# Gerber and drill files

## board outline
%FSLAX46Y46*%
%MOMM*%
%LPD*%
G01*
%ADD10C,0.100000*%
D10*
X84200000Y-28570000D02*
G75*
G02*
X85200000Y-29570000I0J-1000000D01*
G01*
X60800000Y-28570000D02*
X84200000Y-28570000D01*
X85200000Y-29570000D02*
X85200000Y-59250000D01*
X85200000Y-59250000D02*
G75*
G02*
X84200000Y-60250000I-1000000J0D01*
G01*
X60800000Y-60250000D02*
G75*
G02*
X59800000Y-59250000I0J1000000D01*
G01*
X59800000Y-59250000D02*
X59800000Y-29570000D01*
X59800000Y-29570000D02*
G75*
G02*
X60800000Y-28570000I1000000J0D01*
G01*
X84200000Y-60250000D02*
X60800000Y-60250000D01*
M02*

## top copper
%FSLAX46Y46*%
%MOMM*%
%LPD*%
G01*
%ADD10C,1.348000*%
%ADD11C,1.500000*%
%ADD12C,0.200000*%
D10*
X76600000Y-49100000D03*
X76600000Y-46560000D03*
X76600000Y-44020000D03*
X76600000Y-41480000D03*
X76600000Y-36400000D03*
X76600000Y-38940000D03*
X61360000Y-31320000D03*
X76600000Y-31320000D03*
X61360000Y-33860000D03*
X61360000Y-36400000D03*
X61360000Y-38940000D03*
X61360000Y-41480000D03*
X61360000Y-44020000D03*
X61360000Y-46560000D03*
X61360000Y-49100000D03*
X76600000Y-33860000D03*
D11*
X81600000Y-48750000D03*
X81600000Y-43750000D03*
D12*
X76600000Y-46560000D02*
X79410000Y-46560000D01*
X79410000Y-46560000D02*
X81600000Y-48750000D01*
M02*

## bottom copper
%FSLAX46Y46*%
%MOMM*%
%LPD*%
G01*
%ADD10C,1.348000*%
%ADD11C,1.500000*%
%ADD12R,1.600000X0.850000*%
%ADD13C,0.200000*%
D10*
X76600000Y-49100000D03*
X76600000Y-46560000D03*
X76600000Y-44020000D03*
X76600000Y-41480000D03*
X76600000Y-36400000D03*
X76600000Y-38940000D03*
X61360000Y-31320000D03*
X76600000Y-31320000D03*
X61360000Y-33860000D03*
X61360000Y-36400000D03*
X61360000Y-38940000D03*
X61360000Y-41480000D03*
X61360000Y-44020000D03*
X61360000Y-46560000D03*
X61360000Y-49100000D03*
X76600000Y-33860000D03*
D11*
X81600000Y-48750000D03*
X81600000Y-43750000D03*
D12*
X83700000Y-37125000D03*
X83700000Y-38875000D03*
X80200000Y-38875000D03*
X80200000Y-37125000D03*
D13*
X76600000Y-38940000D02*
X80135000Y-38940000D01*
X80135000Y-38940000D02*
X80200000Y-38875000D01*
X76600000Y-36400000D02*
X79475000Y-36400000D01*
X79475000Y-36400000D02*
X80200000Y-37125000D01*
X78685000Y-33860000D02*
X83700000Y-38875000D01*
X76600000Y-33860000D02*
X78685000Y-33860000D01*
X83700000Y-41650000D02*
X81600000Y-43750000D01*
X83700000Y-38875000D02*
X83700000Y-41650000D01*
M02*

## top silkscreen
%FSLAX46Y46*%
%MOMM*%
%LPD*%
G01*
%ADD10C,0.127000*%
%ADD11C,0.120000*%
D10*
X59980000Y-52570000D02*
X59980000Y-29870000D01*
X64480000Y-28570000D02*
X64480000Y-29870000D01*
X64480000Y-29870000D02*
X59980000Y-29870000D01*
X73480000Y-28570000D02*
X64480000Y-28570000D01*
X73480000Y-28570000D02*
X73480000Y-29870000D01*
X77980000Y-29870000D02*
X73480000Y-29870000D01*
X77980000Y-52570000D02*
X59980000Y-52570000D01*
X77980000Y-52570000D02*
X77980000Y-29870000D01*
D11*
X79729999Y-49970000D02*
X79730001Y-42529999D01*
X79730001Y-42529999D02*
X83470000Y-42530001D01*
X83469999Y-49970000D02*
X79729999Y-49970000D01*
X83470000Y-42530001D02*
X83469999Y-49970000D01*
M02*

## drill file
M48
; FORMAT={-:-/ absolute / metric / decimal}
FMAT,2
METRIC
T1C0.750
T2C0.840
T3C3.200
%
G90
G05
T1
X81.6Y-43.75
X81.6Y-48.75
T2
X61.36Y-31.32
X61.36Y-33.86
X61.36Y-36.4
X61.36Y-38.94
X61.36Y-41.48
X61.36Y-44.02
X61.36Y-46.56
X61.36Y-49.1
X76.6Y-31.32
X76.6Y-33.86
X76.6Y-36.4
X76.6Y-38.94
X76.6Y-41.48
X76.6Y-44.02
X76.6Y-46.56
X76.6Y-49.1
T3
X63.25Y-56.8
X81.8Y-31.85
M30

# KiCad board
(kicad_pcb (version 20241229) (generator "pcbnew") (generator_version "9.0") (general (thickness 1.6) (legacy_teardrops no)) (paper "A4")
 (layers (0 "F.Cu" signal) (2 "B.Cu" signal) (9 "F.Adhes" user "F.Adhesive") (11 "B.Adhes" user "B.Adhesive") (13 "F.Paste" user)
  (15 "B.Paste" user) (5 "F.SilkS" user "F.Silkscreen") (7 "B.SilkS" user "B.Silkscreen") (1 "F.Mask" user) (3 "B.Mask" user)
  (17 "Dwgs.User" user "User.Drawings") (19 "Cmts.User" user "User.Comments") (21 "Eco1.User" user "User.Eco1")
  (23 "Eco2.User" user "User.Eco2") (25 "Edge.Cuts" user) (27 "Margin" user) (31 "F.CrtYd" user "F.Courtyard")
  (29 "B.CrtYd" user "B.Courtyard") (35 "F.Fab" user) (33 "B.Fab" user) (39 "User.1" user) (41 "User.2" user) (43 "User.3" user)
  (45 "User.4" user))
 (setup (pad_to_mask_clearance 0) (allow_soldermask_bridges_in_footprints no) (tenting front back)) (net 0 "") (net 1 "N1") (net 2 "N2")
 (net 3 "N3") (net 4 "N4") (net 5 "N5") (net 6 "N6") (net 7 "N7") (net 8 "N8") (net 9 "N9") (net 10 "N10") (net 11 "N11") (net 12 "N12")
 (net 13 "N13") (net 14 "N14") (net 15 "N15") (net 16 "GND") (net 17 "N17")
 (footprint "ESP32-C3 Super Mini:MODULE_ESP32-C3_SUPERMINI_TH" (layer "F.Cu") (at 68.98 41.22)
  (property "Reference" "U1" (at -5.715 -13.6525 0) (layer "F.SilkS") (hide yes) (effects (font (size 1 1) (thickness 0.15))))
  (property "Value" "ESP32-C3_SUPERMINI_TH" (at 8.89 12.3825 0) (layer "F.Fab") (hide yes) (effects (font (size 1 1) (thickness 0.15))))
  (fp_line (start -9 11.35) (end -9 -11.35) (stroke (width 0.127) (type solid)) (layer "F.SilkS"))
  (fp_line (start -4.5 -12.65) (end -4.5 -11.35) (stroke (width 0.127) (type solid)) (layer "F.SilkS"))
  (fp_line (start -4.5 -11.35) (end -9 -11.35) (stroke (width 0.127) (type solid)) (layer "F.SilkS"))
  (fp_line (start 4.5 -12.65) (end -4.5 -12.65) (stroke (width 0.127) (type solid)) (layer "F.SilkS"))
  (fp_line (start 4.5 -12.65) (end 4.5 -11.35) (stroke (width 0.127) (type solid)) (layer "F.SilkS"))
  (fp_line (start 9 -11.35) (end 4.5 -11.35) (stroke (width 0.127) (type solid)) (layer "F.SilkS"))
  (fp_line (start 9 11.35) (end -9 11.35) (stroke (width 0.127) (type solid)) (layer "F.SilkS"))
  (fp_line (start 9 11.35) (end 9 -11.35) (stroke (width 0.127) (type solid)) (layer "F.SilkS"))
  (pad "0" thru_hole circle (at 7.62 7.88) (size 1.348 1.348) (drill 0.84) (layers "*.Cu" "*.Mask") (remove_unused_layers no) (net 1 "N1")
   (solder_mask_margin 0.102))
  (pad "1" thru_hole circle (at 7.62 5.34) (size 1.348 1.348) (drill 0.84) (layers "*.Cu" "*.Mask") (remove_unused_layers no) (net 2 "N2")
   (solder_mask_margin 0.102))
  (pad "2" thru_hole circle (at 7.62 2.8) (size 1.348 1.348) (drill 0.84) (layers "*.Cu" "*.Mask") (remove_unused_layers no) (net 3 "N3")
   (solder_mask_margin 0.102))
  (pad "3" thru_hole circle (at 7.62 0.26) (size 1.348 1.348) (drill 0.84) (layers "*.Cu" "*.Mask") (remove_unused_layers no) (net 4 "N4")
   (solder_mask_margin 0.102))
  (pad "3.3" thru_hole circle (at 7.62 -4.82) (size 1.348 1.348) (drill 0.84) (layers "*.Cu" "*.Mask") (remove_unused_layers no)
   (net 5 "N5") (solder_mask_margin 0.102))
  (pad "4" thru_hole circle (at 7.62 -2.28) (size 1.348 1.348) (drill 0.84) (layers "*.Cu" "*.Mask") (remove_unused_layers no) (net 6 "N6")
   (solder_mask_margin 0.102))
  (pad "5" thru_hole circle (at -7.62 -9.9) (size 1.348 1.348) (drill 0.84) (layers "*.Cu" "*.Mask") (remove_unused_layers no) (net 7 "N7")
   (solder_mask_margin 0.102))
  (pad "5V" thru_hole circle (at 7.62 -9.9) (size 1.348 1.348) (drill 0.84) (layers "*.Cu" "*.Mask") (remove_unused_layers no) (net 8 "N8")
   (solder_mask_margin 0.102))
  (pad "6" thru_hole circle (at -7.62 -7.36) (size 1.348 1.348) (drill 0.84) (layers "*.Cu" "*.Mask") (remove_unused_layers no) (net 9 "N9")
   (solder_mask_margin 0.102))
  (pad "7" thru_hole circle (at -7.62 -4.82) (size 1.348 1.348) (drill 0.84) (layers "*.Cu" "*.Mask") (remove_unused_layers no)
   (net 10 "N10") (solder_mask_margin 0.102))
  (pad "8" thru_hole circle (at -7.62 -2.28) (size 1.348 1.348) (drill 0.84) (layers "*.Cu" "*.Mask") (remove_unused_layers no)
   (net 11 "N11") (solder_mask_margin 0.102))
  (pad "9" thru_hole circle (at -7.62 0.26) (size 1.348 1.348) (drill 0.84) (layers "*.Cu" "*.Mask") (remove_unused_layers no)
   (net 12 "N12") (solder_mask_margin 0.102))
  (pad "10" thru_hole circle (at -7.62 2.8) (size 1.348 1.348) (drill 0.84) (layers "*.Cu" "*.Mask") (remove_unused_layers no)
   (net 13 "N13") (solder_mask_margin 0.102))
  (pad "20" thru_hole circle (at -7.62 5.34) (size 1.348 1.348) (drill 0.84) (layers "*.Cu" "*.Mask") (remove_unused_layers no)
   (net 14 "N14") (solder_mask_margin 0.102))
  (pad "21" thru_hole circle (at -7.62 7.88) (size 1.348 1.348) (drill 0.84) (layers "*.Cu" "*.Mask") (remove_unused_layers no)
   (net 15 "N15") (solder_mask_margin 0.102))
  (pad "G" thru_hole circle (at 7.62 -7.36) (size 1.348 1.348) (drill 0.84) (layers "*.Cu" "*.Mask") (remove_unused_layers no)
   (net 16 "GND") (solder_mask_margin 0.102)))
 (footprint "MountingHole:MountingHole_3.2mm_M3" (layer "F.Cu") (at 81.8 31.85)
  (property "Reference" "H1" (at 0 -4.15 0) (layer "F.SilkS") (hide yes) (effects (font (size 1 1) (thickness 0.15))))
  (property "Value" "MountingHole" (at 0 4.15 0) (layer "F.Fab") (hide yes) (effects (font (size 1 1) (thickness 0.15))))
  (pad "" np_thru_hole circle (at 0 0) (size 3.2 3.2) (drill 3.2) (layers "*.Cu" "*.Mask")))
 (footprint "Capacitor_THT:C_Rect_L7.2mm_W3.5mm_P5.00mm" (layer "F.Cu") (at 81.6 48.75 90)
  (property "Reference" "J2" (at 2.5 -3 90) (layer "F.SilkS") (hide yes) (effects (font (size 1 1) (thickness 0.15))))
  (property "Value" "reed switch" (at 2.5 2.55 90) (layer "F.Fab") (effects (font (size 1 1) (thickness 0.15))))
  (fp_line (start -1.22 -1.870001) (end 6.220001 -1.869999) (stroke (width 0.12) (type solid)) (layer "F.SilkS"))
  (fp_line (start 6.220001 -1.869999) (end 6.219999 1.87) (stroke (width 0.12) (type solid)) (layer "F.SilkS"))
  (fp_line (start -1.22 1.869999) (end -1.22 -1.870001) (stroke (width 0.12) (type solid)) (layer "F.SilkS"))
  (fp_line (start 6.219999 1.87) (end -1.22 1.869999) (stroke (width 0.12) (type solid)) (layer "F.SilkS"))
  (pad "1" thru_hole circle (at 0 0 90) (size 1.5 1.5) (drill 0.75) (layers "*.Cu" "*.Mask") (remove_unused_layers no) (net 2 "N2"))
  (pad "2" thru_hole circle (at 5 0 90) (size 1.5 1.5) (drill 0.75) (layers "*.Cu" "*.Mask") (remove_unused_layers no) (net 16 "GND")))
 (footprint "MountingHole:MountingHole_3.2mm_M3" (layer "F.Cu") (at 63.25 56.8)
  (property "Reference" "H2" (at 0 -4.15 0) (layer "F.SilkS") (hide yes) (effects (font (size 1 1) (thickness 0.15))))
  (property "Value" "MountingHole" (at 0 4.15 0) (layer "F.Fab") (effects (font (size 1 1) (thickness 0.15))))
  (pad "" np_thru_hole circle (at 0 0) (size 3.2 3.2) (drill 3.2) (layers "*.Cu" "*.Mask")))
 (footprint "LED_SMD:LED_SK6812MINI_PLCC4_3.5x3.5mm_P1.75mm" (layer "B.Cu") (at 81.95 38 180)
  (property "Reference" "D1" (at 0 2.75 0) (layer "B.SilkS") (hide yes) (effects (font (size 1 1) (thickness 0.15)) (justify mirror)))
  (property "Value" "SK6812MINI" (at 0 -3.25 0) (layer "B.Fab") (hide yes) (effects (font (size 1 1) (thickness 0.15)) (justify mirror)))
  (pad "1" smd rect (at -1.75 0.875 180) (size 1.6 0.85) (layers "B.Cu" "B.Mask" "B.Paste") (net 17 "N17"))
  (pad "2" smd rect (at -1.75 -0.875 180) (size 1.6 0.85) (layers "B.Cu" "B.Mask" "B.Paste") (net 16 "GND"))
  (pad "3" smd rect (at 1.75 -0.875 180) (size 1.6 0.85) (layers "B.Cu" "B.Mask" "B.Paste") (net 6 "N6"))
  (pad "4" smd rect (at 1.75 0.875 180) (size 1.6 0.85) (layers "B.Cu" "B.Mask" "B.Paste") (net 5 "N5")))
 (gr_arc (start 84.2 28.57) (mid 84.907107 28.862893) (end 85.2 29.57) (stroke (width 0.1) (type solid)) (layer "Edge.Cuts"))
 (gr_line (start 60.8 28.57) (end 84.2 28.57) (stroke (width 0.1) (type solid)) (layer "Edge.Cuts"))
 (gr_line (start 85.2 29.57) (end 85.2 59.25) (stroke (width 0.1) (type solid)) (layer "Edge.Cuts"))
 (gr_arc (start 85.2 59.25) (mid 84.907107 59.957107) (end 84.2 60.25) (stroke (width 0.1) (type solid)) (layer "Edge.Cuts"))
 (gr_arc (start 60.8 60.25) (mid 60.092893 59.957107) (end 59.8 59.25) (stroke (width 0.1) (type solid)) (layer "Edge.Cuts"))
 (gr_line (start 59.8 59.25) (end 59.8 29.57) (stroke (width 0.1) (type solid)) (layer "Edge.Cuts"))
 (gr_arc (start 59.8 29.57) (mid 60.092893 28.862893) (end 60.8 28.57) (stroke (width 0.1) (type solid)) (layer "Edge.Cuts"))
 (gr_line (start 84.2 60.25) (end 60.8 60.25) (stroke (width 0.1) (type solid)) (layer "Edge.Cuts"))
 (segment (start 76.6 38.94) (end 80.135 38.94) (width 0.2) (layer "B.Cu") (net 6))
 (segment (start 80.135 38.94) (end 80.2 38.875) (width 0.2) (layer "B.Cu") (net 6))
 (segment (start 76.6 36.4) (end 79.475 36.4) (width 0.2) (layer "B.Cu") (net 5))
 (segment (start 79.475 36.4) (end 80.2 37.125) (width 0.2) (layer "B.Cu") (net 5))
 (segment (start 78.685 33.86) (end 83.7 38.875) (width 0.2) (layer "B.Cu") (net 16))
 (segment (start 76.6 33.86) (end 78.685 33.86) (width 0.2) (layer "B.Cu") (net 16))
 (segment (start 83.7 41.65) (end 81.6 43.75) (width 0.2) (layer "B.Cu") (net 16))
 (segment (start 83.7 38.875) (end 83.7 41.65) (width 0.2) (layer "B.Cu") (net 16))
 (segment (start 76.6 46.56) (end 79.41 46.56) (width 0.2) (layer "F.Cu") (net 2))
 (segment (start 79.41 46.56) (end 81.6 48.75) (width 0.2) (layer "F.Cu") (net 2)))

